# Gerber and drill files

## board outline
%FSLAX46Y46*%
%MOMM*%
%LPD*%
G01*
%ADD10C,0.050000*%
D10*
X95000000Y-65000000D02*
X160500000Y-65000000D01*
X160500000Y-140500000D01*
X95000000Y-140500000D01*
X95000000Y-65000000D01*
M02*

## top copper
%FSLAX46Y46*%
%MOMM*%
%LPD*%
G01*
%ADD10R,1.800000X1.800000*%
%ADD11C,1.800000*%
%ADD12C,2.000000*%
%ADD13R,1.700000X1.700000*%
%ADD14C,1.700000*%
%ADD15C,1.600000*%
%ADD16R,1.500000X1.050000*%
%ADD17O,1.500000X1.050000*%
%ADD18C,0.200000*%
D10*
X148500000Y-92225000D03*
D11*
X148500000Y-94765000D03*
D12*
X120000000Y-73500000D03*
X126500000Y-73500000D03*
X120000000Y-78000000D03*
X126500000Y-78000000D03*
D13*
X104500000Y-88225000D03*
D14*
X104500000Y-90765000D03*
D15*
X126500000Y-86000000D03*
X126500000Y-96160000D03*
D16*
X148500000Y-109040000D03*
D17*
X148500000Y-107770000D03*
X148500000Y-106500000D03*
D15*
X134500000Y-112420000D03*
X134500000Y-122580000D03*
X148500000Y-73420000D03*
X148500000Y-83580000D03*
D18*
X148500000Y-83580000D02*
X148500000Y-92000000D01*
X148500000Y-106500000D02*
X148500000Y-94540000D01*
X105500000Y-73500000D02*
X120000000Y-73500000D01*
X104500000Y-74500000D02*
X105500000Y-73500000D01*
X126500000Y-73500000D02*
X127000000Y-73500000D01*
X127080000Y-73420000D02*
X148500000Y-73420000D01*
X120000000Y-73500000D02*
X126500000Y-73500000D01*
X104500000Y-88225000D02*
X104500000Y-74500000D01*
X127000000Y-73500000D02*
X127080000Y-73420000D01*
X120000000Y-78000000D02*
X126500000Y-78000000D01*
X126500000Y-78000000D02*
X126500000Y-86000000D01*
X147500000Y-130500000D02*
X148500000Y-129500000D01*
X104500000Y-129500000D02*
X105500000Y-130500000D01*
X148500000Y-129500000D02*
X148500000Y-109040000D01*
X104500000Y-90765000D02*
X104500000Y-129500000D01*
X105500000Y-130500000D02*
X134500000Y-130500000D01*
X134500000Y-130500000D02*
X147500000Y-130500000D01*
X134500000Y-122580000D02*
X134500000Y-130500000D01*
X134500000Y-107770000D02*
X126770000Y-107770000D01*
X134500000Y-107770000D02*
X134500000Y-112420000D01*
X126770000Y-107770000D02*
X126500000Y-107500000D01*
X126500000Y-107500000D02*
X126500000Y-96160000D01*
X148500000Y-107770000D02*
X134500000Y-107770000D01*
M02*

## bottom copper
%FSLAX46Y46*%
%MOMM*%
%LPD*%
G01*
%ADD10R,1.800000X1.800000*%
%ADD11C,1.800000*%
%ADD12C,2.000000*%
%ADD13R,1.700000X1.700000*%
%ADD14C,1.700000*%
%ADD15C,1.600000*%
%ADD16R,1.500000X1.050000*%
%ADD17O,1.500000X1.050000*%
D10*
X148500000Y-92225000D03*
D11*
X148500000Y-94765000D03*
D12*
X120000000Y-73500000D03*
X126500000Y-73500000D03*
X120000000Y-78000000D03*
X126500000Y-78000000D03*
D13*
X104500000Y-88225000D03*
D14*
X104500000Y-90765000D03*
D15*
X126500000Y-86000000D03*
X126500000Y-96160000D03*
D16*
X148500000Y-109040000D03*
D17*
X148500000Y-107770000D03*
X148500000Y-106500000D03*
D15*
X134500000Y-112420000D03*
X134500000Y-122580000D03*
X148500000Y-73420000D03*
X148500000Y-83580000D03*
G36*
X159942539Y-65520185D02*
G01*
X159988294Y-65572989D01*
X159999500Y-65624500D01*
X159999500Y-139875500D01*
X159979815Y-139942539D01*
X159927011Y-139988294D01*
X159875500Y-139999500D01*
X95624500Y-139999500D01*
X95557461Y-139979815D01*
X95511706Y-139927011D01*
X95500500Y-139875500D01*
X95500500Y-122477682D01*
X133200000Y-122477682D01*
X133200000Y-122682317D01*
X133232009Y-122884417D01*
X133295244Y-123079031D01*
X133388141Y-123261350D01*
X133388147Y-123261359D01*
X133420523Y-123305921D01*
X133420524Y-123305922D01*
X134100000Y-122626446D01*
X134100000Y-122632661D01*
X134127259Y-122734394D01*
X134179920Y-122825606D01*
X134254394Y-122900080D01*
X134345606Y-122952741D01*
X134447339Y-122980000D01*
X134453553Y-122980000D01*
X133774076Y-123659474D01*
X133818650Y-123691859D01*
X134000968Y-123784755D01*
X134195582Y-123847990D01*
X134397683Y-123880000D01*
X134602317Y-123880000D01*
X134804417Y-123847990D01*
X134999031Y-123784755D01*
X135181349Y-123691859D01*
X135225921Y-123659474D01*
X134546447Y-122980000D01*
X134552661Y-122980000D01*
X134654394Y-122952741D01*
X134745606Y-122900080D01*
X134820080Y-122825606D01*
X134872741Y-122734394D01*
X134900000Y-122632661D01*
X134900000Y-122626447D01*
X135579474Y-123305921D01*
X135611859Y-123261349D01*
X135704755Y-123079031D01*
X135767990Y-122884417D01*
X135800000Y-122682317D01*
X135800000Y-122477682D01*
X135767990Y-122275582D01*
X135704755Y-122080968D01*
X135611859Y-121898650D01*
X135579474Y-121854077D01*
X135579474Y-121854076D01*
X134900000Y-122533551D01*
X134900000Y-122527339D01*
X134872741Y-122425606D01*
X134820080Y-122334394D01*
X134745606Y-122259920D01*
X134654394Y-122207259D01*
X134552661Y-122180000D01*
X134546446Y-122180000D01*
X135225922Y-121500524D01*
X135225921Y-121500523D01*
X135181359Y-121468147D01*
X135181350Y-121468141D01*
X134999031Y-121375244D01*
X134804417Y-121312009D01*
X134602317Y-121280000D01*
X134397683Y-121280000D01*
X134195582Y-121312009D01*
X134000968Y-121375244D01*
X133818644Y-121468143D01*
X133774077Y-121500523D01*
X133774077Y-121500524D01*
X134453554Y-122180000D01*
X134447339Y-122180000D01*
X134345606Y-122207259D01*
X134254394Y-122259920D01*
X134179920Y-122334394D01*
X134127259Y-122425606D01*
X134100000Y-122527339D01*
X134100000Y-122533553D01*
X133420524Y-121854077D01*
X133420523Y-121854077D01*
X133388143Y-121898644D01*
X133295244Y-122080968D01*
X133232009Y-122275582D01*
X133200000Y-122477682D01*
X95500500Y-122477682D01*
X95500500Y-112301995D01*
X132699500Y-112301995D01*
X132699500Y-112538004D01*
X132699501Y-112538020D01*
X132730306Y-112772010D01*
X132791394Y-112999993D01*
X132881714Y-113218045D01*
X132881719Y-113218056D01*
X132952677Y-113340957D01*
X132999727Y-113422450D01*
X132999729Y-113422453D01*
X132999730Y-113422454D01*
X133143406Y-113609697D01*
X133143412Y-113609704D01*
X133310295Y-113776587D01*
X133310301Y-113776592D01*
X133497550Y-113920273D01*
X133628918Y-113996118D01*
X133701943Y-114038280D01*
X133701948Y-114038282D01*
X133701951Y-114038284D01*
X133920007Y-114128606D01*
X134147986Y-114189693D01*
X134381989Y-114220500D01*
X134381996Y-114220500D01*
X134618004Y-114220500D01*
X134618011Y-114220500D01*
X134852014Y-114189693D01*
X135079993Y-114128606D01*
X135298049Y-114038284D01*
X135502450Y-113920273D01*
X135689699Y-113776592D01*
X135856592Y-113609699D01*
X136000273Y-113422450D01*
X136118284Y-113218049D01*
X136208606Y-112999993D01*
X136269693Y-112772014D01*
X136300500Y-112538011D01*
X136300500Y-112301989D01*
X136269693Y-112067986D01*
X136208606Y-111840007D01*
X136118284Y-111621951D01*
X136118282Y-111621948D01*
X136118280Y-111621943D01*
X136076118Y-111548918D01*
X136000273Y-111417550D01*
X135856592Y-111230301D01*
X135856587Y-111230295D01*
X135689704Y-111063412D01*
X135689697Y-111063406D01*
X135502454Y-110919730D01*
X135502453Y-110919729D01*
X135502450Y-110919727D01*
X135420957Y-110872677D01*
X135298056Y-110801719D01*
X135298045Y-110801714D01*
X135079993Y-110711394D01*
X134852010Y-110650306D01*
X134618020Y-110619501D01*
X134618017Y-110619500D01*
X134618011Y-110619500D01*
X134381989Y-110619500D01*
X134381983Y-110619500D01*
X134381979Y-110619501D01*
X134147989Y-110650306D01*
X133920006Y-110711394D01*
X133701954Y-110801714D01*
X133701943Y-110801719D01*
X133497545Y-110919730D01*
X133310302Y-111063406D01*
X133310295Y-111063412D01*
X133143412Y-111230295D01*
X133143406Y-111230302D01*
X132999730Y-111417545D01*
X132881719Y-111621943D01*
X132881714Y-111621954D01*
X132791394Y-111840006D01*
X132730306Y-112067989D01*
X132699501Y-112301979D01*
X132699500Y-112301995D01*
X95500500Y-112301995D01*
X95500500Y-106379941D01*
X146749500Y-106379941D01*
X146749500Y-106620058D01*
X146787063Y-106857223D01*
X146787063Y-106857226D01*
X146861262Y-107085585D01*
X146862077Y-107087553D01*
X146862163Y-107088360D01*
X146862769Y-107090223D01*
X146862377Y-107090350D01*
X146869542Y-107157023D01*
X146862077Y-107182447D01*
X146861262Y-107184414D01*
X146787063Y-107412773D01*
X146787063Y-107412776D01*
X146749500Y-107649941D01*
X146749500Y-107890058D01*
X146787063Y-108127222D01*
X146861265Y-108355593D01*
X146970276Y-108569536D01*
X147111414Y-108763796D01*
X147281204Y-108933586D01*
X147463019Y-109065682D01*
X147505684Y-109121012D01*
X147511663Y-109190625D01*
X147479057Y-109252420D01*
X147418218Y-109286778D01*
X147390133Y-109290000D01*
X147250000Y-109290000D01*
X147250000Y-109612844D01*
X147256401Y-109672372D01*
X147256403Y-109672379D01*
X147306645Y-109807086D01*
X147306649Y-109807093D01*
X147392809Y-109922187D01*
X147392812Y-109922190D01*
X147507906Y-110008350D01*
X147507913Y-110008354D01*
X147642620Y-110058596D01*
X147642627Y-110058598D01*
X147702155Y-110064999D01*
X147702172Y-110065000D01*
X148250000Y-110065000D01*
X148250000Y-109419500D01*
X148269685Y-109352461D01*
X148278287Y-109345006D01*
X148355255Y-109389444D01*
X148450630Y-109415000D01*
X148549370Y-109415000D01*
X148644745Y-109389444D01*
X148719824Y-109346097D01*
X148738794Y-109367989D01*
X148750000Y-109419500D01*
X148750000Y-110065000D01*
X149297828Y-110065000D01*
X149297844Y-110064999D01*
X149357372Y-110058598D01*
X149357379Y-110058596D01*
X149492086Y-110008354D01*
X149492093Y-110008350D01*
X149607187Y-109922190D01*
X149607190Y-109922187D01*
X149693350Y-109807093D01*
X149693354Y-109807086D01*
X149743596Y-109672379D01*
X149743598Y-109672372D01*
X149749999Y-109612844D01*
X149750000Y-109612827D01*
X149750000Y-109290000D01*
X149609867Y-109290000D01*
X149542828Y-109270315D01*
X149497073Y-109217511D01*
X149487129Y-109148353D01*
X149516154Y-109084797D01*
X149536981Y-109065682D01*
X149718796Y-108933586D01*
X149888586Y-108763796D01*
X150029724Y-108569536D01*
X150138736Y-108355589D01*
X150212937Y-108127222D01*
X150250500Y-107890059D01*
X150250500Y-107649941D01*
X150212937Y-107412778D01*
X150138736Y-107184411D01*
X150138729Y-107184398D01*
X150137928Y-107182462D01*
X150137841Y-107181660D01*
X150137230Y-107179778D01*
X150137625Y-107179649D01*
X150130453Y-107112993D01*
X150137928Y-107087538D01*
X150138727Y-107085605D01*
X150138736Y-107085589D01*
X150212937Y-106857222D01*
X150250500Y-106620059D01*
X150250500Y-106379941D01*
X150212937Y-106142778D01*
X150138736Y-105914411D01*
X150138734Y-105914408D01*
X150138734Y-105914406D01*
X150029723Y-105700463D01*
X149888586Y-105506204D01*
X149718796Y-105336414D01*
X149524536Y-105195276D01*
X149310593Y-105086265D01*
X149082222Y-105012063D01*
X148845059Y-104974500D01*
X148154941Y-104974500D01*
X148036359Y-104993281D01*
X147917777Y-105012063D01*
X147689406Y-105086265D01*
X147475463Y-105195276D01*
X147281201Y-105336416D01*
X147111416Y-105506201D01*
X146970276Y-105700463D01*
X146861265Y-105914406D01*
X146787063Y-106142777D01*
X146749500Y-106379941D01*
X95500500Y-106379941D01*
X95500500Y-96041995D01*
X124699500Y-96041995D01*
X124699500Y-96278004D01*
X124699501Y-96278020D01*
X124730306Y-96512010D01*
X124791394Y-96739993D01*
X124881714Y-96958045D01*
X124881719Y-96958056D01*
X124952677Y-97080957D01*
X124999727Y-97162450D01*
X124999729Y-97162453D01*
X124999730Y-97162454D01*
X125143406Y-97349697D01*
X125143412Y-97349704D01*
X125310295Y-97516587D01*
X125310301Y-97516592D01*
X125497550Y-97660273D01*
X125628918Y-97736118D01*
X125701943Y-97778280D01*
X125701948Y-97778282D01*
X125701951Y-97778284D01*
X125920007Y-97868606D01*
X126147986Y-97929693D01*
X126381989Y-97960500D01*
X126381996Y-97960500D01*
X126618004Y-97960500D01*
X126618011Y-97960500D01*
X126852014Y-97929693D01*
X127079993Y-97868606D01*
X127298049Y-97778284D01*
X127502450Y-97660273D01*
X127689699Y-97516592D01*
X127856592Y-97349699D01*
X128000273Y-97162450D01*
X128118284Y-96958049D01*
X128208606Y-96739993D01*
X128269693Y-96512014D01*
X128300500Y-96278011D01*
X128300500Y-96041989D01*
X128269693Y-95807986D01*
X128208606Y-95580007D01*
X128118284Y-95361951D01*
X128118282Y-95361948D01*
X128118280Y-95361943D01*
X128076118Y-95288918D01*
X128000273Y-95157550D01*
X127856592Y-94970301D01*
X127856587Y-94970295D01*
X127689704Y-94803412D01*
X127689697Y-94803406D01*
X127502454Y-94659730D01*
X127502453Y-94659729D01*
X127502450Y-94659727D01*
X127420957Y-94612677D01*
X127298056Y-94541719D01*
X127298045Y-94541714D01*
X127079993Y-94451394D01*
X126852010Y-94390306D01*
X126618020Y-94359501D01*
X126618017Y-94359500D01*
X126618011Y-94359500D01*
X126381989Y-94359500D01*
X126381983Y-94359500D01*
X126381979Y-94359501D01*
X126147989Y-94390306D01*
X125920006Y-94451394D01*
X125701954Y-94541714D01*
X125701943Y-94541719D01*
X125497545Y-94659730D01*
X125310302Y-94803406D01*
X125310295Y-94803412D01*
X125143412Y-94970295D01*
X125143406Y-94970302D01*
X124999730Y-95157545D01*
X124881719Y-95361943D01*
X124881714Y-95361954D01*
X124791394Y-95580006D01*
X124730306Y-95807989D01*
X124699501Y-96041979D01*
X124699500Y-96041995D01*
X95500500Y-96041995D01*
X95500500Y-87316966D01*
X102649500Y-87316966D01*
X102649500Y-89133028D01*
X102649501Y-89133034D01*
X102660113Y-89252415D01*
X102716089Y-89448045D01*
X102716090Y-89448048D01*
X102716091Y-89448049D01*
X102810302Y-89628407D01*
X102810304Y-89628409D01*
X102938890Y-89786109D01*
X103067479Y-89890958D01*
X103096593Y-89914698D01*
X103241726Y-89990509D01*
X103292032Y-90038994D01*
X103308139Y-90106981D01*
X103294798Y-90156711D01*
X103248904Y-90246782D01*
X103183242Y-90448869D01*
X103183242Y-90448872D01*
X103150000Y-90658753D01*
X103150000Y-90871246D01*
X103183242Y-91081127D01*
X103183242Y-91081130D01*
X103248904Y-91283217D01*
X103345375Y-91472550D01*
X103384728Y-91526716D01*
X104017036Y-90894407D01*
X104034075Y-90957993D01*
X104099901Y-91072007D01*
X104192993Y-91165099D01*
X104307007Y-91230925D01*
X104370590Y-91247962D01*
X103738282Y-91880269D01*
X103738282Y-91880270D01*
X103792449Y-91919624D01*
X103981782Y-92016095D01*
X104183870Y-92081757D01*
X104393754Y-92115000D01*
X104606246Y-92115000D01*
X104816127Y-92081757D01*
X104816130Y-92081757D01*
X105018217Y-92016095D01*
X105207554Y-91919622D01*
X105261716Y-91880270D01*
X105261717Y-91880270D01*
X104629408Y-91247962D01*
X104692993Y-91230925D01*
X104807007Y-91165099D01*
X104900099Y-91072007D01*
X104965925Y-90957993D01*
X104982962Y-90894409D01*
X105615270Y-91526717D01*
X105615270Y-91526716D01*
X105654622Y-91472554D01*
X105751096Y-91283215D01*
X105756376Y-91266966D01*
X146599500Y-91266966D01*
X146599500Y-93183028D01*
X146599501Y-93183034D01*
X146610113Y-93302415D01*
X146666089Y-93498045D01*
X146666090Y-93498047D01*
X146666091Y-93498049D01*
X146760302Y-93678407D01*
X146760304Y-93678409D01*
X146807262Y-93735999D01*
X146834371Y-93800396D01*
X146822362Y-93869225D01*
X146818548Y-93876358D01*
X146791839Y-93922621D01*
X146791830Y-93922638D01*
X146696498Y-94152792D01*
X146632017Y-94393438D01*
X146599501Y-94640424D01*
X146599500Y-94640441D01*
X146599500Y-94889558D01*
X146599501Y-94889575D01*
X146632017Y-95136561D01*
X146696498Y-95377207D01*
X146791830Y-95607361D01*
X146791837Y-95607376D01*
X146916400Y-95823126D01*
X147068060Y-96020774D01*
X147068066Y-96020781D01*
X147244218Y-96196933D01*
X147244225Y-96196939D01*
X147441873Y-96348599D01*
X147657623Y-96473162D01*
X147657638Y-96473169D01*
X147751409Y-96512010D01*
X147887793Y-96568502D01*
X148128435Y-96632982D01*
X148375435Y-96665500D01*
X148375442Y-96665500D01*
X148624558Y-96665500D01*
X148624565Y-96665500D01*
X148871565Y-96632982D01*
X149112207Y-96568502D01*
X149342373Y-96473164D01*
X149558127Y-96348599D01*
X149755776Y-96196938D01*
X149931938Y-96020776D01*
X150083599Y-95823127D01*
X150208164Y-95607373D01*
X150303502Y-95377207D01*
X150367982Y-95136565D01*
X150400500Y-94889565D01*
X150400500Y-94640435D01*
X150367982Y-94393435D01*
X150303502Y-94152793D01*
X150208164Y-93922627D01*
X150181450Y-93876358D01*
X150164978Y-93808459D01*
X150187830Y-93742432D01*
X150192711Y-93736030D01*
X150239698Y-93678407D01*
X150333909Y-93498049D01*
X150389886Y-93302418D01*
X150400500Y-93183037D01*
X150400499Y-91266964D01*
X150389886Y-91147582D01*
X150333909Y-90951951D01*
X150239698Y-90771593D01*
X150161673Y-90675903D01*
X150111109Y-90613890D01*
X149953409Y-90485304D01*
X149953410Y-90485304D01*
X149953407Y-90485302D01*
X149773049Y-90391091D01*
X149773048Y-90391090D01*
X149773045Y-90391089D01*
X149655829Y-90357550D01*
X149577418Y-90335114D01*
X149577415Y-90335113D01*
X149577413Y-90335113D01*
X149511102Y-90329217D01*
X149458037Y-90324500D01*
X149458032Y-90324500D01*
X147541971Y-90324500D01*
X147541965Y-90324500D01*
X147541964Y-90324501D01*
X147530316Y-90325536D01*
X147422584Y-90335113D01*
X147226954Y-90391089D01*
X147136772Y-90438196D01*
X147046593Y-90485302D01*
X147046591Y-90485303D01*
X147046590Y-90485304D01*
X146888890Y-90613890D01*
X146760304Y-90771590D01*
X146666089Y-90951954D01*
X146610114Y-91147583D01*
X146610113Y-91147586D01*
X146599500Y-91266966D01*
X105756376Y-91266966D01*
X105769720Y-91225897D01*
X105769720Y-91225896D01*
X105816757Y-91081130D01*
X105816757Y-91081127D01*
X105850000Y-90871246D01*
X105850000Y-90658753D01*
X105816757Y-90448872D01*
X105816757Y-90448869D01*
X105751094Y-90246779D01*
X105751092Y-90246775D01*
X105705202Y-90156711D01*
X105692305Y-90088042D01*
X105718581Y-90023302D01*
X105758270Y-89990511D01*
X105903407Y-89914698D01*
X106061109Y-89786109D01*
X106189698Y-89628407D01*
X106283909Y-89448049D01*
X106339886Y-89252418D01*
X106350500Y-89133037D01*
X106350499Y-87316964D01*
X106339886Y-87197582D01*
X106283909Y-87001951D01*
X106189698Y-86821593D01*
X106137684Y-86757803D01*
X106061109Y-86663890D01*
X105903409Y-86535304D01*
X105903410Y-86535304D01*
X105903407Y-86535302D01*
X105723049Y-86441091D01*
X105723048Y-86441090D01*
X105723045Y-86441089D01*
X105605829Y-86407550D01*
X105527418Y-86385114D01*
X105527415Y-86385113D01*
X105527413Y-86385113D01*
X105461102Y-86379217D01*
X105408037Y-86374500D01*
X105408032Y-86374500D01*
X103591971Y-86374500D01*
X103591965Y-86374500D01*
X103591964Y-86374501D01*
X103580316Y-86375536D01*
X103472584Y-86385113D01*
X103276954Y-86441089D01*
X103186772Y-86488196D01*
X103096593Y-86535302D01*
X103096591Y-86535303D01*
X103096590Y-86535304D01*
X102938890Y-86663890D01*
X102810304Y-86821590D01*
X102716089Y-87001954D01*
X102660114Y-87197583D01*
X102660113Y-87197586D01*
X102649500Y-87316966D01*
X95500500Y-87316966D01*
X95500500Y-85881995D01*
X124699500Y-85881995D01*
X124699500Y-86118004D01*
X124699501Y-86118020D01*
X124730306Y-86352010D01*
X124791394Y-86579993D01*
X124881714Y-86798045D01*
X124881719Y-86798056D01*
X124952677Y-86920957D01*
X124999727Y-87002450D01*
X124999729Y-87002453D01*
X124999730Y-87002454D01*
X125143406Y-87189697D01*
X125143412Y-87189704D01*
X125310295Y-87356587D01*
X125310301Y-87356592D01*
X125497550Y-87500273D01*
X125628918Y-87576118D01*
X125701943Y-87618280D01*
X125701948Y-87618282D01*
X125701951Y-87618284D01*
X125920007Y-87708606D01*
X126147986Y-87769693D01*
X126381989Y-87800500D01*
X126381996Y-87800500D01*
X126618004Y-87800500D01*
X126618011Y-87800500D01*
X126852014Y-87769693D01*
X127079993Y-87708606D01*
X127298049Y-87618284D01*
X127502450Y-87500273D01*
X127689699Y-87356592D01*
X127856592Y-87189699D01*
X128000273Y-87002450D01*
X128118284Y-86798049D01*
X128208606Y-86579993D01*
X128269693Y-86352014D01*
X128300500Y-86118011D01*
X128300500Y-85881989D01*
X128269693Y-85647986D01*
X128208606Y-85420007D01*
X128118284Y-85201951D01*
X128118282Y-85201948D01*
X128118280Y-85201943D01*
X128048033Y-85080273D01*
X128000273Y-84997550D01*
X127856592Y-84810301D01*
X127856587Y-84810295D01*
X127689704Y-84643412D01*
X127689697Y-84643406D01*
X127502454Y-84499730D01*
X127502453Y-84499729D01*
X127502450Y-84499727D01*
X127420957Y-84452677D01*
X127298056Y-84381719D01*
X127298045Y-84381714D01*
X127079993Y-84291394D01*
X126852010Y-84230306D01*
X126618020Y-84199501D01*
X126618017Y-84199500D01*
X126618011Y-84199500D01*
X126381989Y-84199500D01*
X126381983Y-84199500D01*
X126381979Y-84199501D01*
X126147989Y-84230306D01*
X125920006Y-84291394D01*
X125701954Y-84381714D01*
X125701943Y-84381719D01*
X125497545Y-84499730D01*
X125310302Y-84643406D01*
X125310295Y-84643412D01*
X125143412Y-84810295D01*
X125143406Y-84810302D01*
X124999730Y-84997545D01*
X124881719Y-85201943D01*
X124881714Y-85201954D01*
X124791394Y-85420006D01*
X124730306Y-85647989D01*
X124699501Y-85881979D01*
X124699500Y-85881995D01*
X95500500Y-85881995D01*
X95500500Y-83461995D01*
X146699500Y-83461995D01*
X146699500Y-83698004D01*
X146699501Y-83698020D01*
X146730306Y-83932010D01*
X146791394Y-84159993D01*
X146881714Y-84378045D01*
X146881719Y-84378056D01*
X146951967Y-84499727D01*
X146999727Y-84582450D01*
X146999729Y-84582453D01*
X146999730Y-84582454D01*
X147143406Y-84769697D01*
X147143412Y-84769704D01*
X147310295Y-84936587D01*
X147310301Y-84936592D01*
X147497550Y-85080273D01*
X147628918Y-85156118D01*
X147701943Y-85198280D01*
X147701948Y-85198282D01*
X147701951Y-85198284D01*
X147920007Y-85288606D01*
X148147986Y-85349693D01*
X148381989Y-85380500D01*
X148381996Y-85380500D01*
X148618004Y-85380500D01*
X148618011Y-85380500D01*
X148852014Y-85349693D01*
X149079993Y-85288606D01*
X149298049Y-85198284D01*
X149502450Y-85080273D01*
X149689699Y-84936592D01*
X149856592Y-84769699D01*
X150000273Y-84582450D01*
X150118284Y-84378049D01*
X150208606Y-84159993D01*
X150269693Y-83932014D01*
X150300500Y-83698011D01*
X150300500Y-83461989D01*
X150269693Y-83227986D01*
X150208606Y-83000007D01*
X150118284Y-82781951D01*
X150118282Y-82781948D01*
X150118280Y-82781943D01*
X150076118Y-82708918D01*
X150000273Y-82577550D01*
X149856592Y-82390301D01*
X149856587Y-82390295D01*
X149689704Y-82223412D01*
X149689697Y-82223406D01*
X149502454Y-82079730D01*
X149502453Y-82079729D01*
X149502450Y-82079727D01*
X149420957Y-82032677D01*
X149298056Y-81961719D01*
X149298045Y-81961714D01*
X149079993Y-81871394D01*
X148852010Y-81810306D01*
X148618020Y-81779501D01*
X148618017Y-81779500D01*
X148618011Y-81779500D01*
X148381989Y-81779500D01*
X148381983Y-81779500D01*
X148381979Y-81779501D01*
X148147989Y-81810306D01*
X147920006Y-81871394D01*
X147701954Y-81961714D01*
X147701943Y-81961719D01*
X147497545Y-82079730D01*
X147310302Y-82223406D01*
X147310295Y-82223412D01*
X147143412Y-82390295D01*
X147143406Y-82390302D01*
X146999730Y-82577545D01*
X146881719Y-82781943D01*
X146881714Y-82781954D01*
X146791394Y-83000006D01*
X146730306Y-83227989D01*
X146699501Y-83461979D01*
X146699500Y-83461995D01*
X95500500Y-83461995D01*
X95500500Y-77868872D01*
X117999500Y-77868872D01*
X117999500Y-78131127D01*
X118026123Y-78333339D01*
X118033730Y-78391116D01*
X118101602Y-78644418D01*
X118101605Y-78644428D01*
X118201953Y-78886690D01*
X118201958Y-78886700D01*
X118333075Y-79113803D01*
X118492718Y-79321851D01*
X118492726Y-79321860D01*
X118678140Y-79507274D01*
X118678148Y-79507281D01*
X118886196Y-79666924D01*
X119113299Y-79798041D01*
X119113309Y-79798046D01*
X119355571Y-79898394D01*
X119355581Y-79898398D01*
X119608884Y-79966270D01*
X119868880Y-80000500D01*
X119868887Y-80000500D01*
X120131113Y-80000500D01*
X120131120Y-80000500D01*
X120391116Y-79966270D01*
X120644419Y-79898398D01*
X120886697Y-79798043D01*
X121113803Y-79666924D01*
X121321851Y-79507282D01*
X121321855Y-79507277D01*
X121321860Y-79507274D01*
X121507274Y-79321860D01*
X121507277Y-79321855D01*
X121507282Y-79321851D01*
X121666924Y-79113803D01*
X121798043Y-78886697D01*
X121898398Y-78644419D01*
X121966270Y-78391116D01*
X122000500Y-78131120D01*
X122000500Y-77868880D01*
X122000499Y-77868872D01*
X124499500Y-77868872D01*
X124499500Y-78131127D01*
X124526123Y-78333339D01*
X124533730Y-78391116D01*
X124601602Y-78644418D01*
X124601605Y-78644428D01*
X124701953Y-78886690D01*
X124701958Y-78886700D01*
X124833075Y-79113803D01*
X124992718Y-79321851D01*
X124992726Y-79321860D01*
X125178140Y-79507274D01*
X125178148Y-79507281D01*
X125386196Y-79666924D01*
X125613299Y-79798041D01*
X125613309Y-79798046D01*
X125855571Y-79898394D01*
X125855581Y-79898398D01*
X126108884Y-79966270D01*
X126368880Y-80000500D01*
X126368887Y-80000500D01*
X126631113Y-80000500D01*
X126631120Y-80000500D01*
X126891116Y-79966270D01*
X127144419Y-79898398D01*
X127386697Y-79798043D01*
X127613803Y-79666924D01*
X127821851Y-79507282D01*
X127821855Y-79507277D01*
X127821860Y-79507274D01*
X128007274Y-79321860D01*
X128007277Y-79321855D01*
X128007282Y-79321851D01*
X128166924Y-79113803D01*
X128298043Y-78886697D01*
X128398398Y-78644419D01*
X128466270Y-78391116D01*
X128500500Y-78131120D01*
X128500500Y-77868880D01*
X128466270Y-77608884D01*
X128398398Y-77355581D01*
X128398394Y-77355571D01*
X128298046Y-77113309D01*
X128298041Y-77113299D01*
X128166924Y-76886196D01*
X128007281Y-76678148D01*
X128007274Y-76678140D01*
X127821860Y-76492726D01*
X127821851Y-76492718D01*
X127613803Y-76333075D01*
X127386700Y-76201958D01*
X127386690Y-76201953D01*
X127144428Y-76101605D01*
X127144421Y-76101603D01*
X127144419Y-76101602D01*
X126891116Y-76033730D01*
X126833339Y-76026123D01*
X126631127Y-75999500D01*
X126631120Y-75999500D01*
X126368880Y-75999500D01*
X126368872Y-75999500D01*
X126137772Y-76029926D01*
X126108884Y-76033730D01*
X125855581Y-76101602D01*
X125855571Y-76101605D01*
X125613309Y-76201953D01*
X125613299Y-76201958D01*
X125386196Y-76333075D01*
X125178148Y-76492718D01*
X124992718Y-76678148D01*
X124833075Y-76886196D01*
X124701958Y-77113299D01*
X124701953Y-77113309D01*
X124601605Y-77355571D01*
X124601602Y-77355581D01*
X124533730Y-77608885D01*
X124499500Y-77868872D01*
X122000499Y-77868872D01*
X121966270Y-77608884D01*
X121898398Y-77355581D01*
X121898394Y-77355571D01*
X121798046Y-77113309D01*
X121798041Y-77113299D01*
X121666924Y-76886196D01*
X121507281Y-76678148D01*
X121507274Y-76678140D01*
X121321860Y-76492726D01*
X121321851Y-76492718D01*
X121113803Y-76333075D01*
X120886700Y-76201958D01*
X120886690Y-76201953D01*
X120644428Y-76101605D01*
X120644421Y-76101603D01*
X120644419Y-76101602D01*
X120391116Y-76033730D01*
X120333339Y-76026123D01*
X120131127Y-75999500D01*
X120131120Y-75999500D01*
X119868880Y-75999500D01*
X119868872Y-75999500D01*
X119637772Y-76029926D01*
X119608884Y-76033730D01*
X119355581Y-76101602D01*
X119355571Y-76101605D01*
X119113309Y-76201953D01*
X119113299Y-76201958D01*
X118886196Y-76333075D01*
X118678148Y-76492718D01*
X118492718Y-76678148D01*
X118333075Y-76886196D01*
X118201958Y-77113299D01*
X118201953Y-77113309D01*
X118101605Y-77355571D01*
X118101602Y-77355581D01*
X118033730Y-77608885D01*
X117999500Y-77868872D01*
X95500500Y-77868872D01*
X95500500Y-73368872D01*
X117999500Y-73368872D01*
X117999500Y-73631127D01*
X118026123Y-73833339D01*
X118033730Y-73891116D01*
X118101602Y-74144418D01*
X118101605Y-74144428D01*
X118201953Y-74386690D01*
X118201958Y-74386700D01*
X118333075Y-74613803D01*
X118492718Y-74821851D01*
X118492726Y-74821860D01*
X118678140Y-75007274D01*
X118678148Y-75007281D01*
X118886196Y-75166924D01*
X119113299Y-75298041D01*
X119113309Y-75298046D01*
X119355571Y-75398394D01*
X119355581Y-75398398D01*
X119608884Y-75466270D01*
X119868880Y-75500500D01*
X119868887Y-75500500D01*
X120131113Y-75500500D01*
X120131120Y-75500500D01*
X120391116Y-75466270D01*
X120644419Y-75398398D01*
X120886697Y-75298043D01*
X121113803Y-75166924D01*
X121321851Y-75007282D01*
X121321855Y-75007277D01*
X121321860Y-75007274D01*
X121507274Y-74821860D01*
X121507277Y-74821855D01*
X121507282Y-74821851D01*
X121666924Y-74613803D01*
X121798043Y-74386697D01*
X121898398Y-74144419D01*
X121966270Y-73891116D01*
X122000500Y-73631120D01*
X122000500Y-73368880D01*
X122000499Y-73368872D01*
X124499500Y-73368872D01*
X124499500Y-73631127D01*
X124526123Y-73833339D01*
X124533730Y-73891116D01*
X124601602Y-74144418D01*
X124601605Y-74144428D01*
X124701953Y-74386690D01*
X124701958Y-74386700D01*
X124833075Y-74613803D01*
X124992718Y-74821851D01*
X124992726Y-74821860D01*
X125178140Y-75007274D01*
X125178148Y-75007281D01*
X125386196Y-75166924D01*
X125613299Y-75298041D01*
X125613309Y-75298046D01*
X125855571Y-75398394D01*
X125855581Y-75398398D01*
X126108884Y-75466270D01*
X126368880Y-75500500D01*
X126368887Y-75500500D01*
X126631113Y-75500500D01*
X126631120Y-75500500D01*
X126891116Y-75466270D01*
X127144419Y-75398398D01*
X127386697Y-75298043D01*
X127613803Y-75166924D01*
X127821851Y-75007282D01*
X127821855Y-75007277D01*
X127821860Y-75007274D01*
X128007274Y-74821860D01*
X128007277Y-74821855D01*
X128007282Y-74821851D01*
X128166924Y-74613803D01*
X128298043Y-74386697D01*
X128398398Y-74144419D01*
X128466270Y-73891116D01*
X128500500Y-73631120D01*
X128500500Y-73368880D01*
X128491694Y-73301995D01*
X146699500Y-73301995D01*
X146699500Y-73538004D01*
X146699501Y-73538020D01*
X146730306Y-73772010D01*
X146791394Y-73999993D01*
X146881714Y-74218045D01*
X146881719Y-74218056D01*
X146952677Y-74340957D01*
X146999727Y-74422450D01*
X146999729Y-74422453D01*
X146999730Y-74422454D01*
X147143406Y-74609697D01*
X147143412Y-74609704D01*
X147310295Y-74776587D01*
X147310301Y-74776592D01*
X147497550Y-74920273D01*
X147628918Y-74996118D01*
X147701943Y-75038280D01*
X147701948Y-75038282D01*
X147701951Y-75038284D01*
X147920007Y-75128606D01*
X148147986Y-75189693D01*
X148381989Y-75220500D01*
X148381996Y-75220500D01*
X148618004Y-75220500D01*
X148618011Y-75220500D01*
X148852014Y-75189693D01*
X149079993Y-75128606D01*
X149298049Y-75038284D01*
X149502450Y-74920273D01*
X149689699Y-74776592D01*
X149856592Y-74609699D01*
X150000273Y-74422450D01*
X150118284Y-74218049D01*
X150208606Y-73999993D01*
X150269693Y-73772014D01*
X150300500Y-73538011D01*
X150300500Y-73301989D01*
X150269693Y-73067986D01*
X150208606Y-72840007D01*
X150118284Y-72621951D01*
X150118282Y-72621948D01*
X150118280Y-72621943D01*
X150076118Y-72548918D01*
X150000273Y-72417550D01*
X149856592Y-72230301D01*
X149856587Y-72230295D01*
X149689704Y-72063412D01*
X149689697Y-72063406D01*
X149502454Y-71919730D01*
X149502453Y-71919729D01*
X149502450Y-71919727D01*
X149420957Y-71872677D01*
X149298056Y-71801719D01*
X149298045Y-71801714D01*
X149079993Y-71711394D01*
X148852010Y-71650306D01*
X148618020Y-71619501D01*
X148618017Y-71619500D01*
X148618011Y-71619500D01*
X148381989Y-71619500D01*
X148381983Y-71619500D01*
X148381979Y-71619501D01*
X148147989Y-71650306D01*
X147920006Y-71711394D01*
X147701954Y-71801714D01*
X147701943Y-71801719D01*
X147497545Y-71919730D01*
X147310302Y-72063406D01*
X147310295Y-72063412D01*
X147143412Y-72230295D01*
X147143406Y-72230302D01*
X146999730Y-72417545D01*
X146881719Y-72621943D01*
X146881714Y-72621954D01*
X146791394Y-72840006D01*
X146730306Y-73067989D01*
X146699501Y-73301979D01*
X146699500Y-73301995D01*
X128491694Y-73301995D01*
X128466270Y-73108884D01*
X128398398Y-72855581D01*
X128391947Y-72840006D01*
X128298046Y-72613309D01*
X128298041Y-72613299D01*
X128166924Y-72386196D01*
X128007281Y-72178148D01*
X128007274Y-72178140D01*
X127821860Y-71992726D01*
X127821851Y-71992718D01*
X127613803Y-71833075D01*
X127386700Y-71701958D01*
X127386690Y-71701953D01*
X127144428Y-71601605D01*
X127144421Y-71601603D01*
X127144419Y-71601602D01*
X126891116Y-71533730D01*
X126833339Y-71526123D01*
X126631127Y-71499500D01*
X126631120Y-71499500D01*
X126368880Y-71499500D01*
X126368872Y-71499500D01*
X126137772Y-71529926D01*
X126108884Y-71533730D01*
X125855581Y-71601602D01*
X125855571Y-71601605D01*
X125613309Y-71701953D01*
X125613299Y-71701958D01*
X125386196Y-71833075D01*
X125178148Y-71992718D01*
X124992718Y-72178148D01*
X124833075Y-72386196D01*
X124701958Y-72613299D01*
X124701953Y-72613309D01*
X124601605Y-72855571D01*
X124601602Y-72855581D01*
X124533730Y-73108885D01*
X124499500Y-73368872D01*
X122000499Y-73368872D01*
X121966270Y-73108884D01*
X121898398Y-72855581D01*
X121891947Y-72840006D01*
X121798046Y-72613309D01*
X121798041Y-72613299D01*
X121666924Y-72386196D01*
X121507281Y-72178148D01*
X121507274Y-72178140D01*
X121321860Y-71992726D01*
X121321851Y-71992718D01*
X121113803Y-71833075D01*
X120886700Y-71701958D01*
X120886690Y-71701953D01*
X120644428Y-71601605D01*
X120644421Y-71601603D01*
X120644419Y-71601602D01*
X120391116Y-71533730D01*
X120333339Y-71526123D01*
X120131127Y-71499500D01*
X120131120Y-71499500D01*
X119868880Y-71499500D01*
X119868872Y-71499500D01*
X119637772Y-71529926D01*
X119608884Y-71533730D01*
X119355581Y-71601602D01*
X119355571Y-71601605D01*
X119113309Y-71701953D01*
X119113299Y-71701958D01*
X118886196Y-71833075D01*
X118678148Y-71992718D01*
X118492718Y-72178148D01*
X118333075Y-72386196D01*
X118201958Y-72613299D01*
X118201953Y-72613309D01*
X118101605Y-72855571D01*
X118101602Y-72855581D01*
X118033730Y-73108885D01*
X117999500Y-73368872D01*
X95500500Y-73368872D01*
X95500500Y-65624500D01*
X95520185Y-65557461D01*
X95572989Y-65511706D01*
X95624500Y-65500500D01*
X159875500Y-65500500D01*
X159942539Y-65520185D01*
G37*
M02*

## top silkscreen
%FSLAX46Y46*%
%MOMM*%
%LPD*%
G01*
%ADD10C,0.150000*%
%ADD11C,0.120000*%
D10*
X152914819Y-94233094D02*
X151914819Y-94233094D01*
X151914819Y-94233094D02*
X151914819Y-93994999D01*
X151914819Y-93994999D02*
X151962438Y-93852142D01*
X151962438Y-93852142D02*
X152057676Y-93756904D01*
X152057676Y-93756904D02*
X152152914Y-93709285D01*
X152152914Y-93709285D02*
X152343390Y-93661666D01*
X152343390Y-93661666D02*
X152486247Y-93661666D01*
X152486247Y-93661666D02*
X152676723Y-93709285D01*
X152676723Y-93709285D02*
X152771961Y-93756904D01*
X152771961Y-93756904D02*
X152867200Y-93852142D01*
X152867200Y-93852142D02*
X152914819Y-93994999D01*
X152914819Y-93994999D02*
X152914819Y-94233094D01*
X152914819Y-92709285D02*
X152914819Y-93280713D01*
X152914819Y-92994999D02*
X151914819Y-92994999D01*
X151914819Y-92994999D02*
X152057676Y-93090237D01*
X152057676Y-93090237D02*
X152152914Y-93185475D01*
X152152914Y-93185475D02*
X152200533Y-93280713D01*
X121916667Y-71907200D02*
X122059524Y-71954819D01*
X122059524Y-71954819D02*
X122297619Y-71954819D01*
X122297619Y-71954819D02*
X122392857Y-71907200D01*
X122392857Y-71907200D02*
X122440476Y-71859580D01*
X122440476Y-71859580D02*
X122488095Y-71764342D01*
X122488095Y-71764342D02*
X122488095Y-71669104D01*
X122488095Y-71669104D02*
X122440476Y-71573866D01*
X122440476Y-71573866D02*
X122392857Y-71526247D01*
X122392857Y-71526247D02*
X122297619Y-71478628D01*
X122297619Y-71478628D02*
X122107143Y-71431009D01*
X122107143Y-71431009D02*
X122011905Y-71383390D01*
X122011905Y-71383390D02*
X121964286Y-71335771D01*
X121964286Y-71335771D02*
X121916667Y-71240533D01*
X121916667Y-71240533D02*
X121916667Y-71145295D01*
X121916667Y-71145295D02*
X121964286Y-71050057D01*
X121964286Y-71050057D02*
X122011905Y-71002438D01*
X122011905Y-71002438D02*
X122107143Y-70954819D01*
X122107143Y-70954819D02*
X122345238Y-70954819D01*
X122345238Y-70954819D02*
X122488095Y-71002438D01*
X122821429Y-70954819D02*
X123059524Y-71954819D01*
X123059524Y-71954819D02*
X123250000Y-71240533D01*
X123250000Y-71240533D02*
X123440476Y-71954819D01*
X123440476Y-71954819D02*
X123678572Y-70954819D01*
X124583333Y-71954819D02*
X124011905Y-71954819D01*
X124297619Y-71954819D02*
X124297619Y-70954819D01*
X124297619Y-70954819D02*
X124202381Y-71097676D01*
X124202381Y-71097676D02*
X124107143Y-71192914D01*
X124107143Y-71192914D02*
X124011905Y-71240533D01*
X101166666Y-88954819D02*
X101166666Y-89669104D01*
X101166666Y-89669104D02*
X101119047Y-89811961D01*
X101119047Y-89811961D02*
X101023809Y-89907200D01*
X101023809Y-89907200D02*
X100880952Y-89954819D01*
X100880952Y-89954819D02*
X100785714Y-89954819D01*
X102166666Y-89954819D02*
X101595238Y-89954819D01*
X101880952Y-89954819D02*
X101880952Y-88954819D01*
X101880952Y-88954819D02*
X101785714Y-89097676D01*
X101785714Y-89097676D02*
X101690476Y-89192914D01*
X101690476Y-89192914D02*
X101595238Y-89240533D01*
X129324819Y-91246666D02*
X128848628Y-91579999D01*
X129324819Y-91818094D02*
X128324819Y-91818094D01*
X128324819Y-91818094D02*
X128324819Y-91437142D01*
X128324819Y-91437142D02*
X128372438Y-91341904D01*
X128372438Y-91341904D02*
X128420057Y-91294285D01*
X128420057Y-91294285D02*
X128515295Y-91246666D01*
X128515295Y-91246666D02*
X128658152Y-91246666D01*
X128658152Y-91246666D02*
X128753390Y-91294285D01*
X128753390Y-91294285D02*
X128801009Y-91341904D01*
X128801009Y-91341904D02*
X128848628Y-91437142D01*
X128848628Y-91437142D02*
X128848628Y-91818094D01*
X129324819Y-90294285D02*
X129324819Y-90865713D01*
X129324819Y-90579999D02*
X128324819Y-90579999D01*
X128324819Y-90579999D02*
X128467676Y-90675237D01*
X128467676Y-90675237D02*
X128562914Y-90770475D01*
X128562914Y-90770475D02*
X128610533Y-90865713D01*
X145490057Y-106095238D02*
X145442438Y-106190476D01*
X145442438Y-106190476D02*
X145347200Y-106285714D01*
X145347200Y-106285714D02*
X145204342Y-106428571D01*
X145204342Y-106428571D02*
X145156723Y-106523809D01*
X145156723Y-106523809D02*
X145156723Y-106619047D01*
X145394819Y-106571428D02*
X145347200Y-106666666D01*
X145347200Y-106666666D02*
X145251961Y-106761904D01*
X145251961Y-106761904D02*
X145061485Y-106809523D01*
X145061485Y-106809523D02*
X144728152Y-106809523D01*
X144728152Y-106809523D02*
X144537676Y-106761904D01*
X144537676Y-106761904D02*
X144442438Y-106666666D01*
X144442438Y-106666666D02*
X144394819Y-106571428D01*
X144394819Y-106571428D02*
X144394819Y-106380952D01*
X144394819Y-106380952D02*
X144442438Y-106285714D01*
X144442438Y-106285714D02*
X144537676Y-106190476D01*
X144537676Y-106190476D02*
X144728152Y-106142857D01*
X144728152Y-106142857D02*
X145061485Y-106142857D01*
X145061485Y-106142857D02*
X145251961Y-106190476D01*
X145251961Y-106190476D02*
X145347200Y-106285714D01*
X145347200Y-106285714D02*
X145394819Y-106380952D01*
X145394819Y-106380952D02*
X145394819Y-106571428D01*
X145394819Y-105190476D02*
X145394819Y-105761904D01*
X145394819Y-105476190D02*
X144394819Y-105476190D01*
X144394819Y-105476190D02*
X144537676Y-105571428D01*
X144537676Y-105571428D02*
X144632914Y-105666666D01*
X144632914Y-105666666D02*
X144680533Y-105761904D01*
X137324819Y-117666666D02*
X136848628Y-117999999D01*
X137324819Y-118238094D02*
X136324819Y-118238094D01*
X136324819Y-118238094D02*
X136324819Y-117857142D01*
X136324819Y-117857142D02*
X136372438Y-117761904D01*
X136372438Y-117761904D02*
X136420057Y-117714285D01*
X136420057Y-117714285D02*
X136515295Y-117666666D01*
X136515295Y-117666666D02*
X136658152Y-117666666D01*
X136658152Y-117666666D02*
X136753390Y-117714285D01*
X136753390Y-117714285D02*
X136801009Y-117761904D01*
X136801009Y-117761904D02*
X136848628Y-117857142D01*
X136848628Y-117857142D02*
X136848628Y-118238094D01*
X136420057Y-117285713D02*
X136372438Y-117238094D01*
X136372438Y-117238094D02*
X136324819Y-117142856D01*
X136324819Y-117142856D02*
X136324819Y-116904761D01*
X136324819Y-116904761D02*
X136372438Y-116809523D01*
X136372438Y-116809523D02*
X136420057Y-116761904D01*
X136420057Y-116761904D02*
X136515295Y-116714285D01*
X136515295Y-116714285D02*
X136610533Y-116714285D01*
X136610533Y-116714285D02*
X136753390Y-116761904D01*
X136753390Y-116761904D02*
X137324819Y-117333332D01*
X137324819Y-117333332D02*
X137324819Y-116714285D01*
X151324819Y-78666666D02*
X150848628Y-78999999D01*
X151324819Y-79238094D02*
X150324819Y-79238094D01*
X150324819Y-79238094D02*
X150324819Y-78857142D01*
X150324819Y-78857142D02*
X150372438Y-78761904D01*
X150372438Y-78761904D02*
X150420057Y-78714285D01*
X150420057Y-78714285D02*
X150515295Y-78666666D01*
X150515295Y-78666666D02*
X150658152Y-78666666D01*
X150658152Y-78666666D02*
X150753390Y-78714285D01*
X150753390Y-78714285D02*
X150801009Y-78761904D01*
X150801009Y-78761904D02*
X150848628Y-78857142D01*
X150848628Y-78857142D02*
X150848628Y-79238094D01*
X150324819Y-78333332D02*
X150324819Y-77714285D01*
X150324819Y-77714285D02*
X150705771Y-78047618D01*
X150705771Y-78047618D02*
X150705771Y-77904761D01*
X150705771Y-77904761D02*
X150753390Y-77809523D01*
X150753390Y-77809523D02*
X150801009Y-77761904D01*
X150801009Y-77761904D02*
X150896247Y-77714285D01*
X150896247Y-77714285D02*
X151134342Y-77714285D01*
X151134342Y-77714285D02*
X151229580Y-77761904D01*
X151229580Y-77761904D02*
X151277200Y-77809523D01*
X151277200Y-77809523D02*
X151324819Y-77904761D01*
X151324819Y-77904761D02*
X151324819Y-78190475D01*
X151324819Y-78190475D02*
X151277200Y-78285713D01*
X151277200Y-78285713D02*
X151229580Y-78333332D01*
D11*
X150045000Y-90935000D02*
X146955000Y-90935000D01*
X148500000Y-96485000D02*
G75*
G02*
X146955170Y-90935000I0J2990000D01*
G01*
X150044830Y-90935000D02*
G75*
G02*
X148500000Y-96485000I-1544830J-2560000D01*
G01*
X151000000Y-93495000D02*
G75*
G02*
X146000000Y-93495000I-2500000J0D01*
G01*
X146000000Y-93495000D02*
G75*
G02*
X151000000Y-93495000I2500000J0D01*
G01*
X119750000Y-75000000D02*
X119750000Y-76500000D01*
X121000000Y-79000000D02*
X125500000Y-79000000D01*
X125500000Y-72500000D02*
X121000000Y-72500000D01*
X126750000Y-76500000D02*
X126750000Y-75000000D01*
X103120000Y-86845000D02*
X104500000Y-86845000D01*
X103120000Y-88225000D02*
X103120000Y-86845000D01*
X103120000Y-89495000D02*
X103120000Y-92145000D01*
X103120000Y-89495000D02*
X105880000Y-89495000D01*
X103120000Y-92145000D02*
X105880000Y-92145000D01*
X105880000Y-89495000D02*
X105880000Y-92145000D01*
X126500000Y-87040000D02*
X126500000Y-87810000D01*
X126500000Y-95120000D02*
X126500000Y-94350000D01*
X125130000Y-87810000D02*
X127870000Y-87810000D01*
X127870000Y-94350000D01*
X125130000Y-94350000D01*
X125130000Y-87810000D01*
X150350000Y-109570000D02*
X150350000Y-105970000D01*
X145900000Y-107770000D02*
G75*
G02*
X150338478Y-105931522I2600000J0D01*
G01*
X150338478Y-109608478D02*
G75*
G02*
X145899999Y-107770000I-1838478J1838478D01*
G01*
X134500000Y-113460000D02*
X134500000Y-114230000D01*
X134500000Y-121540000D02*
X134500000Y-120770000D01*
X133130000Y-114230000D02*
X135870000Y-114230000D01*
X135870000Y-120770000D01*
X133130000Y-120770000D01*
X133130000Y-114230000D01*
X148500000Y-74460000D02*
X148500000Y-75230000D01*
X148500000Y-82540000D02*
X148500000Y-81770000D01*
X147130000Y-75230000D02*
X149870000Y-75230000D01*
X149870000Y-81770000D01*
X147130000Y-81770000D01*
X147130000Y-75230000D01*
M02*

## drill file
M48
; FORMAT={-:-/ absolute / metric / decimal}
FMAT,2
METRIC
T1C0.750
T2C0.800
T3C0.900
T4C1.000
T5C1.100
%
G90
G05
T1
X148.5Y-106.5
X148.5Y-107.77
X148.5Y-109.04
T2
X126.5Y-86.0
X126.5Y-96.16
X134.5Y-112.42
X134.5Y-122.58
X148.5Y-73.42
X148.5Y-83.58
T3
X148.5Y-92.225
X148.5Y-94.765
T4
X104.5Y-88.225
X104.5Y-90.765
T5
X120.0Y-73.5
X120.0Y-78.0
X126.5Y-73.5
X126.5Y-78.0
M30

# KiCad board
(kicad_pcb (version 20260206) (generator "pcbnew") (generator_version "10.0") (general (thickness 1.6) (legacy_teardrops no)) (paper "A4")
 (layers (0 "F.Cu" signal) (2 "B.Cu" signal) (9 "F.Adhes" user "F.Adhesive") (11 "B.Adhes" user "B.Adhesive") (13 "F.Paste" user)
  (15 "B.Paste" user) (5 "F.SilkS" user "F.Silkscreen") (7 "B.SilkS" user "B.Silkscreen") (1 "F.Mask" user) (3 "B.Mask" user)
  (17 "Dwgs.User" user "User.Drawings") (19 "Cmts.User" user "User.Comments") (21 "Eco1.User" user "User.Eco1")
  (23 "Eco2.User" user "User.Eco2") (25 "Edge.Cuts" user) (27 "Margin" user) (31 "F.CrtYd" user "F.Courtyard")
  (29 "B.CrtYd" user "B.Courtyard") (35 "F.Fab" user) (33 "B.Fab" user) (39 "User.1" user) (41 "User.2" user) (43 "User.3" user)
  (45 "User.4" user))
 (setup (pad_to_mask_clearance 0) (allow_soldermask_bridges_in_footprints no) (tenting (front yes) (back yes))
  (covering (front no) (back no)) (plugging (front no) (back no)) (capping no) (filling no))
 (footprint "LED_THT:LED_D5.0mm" (layer "F.Cu") (at 148.5 92.225 -90)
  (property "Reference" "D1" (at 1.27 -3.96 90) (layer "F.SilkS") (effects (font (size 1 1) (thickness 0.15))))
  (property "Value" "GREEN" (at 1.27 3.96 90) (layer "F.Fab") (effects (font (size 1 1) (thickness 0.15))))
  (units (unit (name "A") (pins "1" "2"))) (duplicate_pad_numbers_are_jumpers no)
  (fp_line (start -1.29 -1.545) (end -1.29 1.545) (stroke (width 0.12) (type solid)) (layer "F.SilkS"))
  (fp_arc (start 4.26 0) (mid 2.071779 2.880495) (end -1.29 1.54483) (stroke (width 0.12) (type solid)) (layer "F.SilkS"))
  (fp_arc (start -1.29 -1.54483) (mid 2.071779 -2.880495) (end 4.26 0) (stroke (width 0.12) (type solid)) (layer "F.SilkS"))
  (fp_circle (center 1.27 0) (end 3.77 0) (stroke (width 0.12) (type solid)) (fill no) (layer "F.SilkS"))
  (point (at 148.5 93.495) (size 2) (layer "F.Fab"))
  (pad "1" thru_hole rect (at 0 0 270) (size 1.8 1.8) (drill 0.9) (layers "*.Cu" "*.Mask") (remove_unused_layers no) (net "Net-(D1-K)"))
  (pad "2" thru_hole circle (at 2.54 0 270) (size 1.8 1.8) (drill 0.9) (layers "*.Cu" "*.Mask") (remove_unused_layers no) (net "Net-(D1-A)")))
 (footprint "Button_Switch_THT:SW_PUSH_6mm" (layer "F.Cu") (at 120 73.5)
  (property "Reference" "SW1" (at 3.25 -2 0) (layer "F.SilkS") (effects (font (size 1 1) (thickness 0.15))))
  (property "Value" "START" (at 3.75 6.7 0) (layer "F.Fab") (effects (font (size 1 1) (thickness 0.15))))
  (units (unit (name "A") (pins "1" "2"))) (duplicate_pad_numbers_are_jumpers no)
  (fp_line (start -0.25 1.5) (end -0.25 3) (stroke (width 0.12) (type solid)) (layer "F.SilkS"))
  (fp_line (start 1 5.5) (end 5.5 5.5) (stroke (width 0.12) (type solid)) (layer "F.SilkS"))
  (fp_line (start 5.5 -1) (end 1 -1) (stroke (width 0.12) (type solid)) (layer "F.SilkS"))
  (fp_line (start 6.75 3) (end 6.75 1.5) (stroke (width 0.12) (type solid)) (layer "F.SilkS"))
  (pad "1" thru_hole circle (at 0 0 90) (size 2 2) (drill 1.1) (layers "*.Cu" "*.Mask") (remove_unused_layers no) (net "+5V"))
  (pad "1" thru_hole circle (at 6.5 0 90) (size 2 2) (drill 1.1) (layers "*.Cu" "*.Mask") (remove_unused_layers no) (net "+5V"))
  (pad "2" thru_hole circle (at 0 4.5 90) (size 2 2) (drill 1.1) (layers "*.Cu" "*.Mask") (remove_unused_layers no) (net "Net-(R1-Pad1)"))
  (pad "2" thru_hole circle (at 6.5 4.5 90) (size 2 2) (drill 1.1) (layers "*.Cu" "*.Mask") (remove_unused_layers no) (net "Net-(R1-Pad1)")))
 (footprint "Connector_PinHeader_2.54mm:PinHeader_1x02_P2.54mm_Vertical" (layer "F.Cu") (at 104.5 88.225)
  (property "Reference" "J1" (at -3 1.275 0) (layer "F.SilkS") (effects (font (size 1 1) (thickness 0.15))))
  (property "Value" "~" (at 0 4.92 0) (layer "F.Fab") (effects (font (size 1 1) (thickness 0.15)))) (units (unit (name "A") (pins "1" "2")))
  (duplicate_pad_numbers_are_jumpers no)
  (fp_line (start -1.38 -1.38) (end 0 -1.38) (stroke (width 0.12) (type solid)) (layer "F.SilkS"))
  (fp_line (start -1.38 0) (end -1.38 -1.38) (stroke (width 0.12) (type solid)) (layer "F.SilkS"))
  (fp_line (start -1.38 1.27) (end -1.38 3.92) (stroke (width 0.12) (type solid)) (layer "F.SilkS"))
  (fp_line (start -1.38 1.27) (end 1.38 1.27) (stroke (width 0.12) (type solid)) (layer "F.SilkS"))
  (fp_line (start -1.38 3.92) (end 1.38 3.92) (stroke (width 0.12) (type solid)) (layer "F.SilkS"))
  (fp_line (start 1.38 1.27) (end 1.38 3.92) (stroke (width 0.12) (type solid)) (layer "F.SilkS"))
  (pad "1" thru_hole rect (at 0 0) (size 1.7 1.7) (drill 1) (layers "*.Cu" "*.Mask") (remove_unused_layers no) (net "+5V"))
  (pad "2" thru_hole circle (at 0 2.54) (size 1.7 1.7) (drill 1) (layers "*.Cu" "*.Mask") (remove_unused_layers no) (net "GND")))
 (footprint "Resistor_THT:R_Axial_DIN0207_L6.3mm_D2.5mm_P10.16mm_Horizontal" (layer "F.Cu") (at 126.5 86 -90)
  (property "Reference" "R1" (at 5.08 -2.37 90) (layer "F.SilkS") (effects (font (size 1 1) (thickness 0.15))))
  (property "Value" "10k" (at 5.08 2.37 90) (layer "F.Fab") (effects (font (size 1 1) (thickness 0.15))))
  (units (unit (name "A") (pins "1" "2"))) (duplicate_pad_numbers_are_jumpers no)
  (fp_line (start 1.04 0) (end 1.81 0) (stroke (width 0.12) (type solid)) (layer "F.SilkS"))
  (fp_line (start 9.12 0) (end 8.35 0) (stroke (width 0.12) (type solid)) (layer "F.SilkS"))
  (fp_rect (start 1.81 -1.37) (end 8.35 1.37) (stroke (width 0.12) (type solid)) (fill no) (layer "F.SilkS"))
  (pad "1" thru_hole circle (at 0 0 270) (size 1.6 1.6) (drill 0.8) (layers "*.Cu" "*.Mask") (remove_unused_layers no) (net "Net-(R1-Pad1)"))
  (pad "2" thru_hole circle (at 10.16 0 270) (size 1.6 1.6) (drill 0.8) (layers "*.Cu" "*.Mask") (remove_unused_layers no) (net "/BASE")))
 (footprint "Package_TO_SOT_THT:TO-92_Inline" (layer "F.Cu") (at 148.5 109.04 90)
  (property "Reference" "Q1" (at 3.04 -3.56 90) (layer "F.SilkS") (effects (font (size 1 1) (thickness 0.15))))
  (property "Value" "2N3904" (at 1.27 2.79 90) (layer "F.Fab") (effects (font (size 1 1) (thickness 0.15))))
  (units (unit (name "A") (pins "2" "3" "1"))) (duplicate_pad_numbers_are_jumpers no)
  (fp_line (start -0.53 1.85) (end 3.07 1.85) (stroke (width 0.12) (type solid)) (layer "F.SilkS"))
  (fp_arc (start 1.27 -2.6) (mid 3.672087 -0.994977) (end 3.108478 1.838478) (stroke (width 0.12) (type solid)) (layer "F.SilkS"))
  (fp_arc (start -0.568478 1.838478) (mid -1.132087 -0.994977) (end 1.27 -2.6) (stroke (width 0.12) (type solid)) (layer "F.SilkS"))
  (pad "1" thru_hole rect (at 0 0 90) (size 1.05 1.5) (drill 0.75) (layers "*.Cu" "*.Mask") (remove_unused_layers no) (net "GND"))
  (pad "2" thru_hole oval (at 1.27 0 90) (size 1.05 1.5) (drill 0.75) (layers "*.Cu" "*.Mask") (remove_unused_layers no) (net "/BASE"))
  (pad "3" thru_hole oval (at 2.54 0 90) (size 1.05 1.5) (drill 0.75) (layers "*.Cu" "*.Mask") (remove_unused_layers no) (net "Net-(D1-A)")))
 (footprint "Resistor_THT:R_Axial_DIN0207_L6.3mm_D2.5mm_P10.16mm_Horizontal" (layer "F.Cu") (at 134.5 112.42 -90)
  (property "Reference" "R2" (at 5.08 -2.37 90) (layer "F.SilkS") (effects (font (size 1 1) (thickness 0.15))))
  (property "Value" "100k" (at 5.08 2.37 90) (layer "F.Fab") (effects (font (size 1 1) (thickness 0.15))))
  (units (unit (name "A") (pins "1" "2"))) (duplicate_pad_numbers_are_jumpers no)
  (fp_line (start 1.04 0) (end 1.81 0) (stroke (width 0.12) (type solid)) (layer "F.SilkS"))
  (fp_line (start 9.12 0) (end 8.35 0) (stroke (width 0.12) (type solid)) (layer "F.SilkS"))
  (fp_rect (start 1.81 -1.37) (end 8.35 1.37) (stroke (width 0.12) (type solid)) (fill no) (layer "F.SilkS"))
  (pad "1" thru_hole circle (at 0 0 270) (size 1.6 1.6) (drill 0.8) (layers "*.Cu" "*.Mask") (remove_unused_layers no) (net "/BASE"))
  (pad "2" thru_hole circle (at 10.16 0 270) (size 1.6 1.6) (drill 0.8) (layers "*.Cu" "*.Mask") (remove_unused_layers no) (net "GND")))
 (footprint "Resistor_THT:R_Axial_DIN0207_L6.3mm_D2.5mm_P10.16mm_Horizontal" (layer "F.Cu") (at 148.5 73.42 -90)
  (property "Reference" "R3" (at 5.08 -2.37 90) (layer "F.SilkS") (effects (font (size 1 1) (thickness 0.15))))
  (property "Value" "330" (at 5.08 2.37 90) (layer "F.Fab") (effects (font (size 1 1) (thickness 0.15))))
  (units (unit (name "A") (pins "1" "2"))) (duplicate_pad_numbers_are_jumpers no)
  (fp_line (start 1.04 0) (end 1.81 0) (stroke (width 0.12) (type solid)) (layer "F.SilkS"))
  (fp_line (start 9.12 0) (end 8.35 0) (stroke (width 0.12) (type solid)) (layer "F.SilkS"))
  (fp_rect (start 1.81 -1.37) (end 8.35 1.37) (stroke (width 0.12) (type solid)) (fill no) (layer "F.SilkS"))
  (pad "1" thru_hole circle (at 0 0 270) (size 1.6 1.6) (drill 0.8) (layers "*.Cu" "*.Mask") (remove_unused_layers no) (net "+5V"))
  (pad "2" thru_hole circle (at 10.16 0 270) (size 1.6 1.6) (drill 0.8) (layers "*.Cu" "*.Mask") (remove_unused_layers no)
   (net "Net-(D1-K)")))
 (gr_rect (start 95 65) (end 160.5 140.5) (stroke (width 0.05) (type default)) (fill no) (layer "Edge.Cuts"))
 (segment (start 148.5 83.58) (end 148.5 92) (width 0.2) (layers "F.Cu" "F.Mask") (solder_mask_margin 0.2) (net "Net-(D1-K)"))
 (segment (start 148.5 106.5) (end 148.5 94.54) (width 0.2) (layers "F.Cu" "F.Mask") (solder_mask_margin 0.2) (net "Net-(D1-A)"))
 (segment (start 105.5 73.5) (end 120 73.5) (width 0.2) (layers "F.Cu" "F.Mask") (solder_mask_margin 0.2) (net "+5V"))
 (segment (start 104.5 74.5) (end 105.5 73.5) (width 0.2) (layers "F.Cu" "F.Mask") (solder_mask_margin 0.2) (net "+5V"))
 (segment (start 126.5 73.5) (end 127 73.5) (width 0.2) (layers "F.Cu" "F.Mask") (solder_mask_margin 0.2) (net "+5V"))
 (segment (start 127.08 73.42) (end 148.5 73.42) (width 0.2) (layers "F.Cu" "F.Mask") (solder_mask_margin 0.2) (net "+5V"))
 (segment (start 120 73.5) (end 126.5 73.5) (width 0.2) (layers "F.Cu" "F.Mask") (solder_mask_margin 0.2) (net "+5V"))
 (segment (start 104.5 88.225) (end 104.5 74.5) (width 0.2) (layers "F.Cu" "F.Mask") (solder_mask_margin 0.2) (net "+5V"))
 (segment (start 127 73.5) (end 127.08 73.42) (width 0.2) (layers "F.Cu" "F.Mask") (solder_mask_margin 0.2) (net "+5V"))
 (segment (start 120 78) (end 126.5 78) (width 0.2) (layers "F.Cu" "F.Mask") (solder_mask_margin 0.2) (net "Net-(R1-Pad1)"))
 (segment (start 126.5 78) (end 126.5 86) (width 0.2) (layers "F.Cu" "F.Mask") (solder_mask_margin 0.2) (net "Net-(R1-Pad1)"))
 (segment (start 147.5 130.5) (end 148.5 129.5) (width 0.2) (layers "F.Cu" "F.Mask") (solder_mask_margin 0.2) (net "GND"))
 (segment (start 104.5 129.5) (end 105.5 130.5) (width 0.2) (layers "F.Cu" "F.Mask") (solder_mask_margin 0.2) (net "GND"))
 (segment (start 148.5 129.5) (end 148.5 109.04) (width 0.2) (layers "F.Cu" "F.Mask") (solder_mask_margin 0.2) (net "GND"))
 (segment (start 104.5 90.765) (end 104.5 129.5) (width 0.2) (layers "F.Cu" "F.Mask") (solder_mask_margin 0.2) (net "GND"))
 (segment (start 105.5 130.5) (end 134.5 130.5) (width 0.2) (layers "F.Cu" "F.Mask") (solder_mask_margin 0.2) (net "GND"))
 (segment (start 134.5 130.5) (end 147.5 130.5) (width 0.2) (layers "F.Cu" "F.Mask") (solder_mask_margin 0.2) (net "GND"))
 (segment (start 134.5 122.58) (end 134.5 130.5) (width 0.2) (layers "F.Cu" "F.Mask") (solder_mask_margin 0.2) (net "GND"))
 (segment (start 134.5 107.77) (end 126.77 107.77) (width 0.2) (layers "F.Cu" "F.Mask") (solder_mask_margin 0.2) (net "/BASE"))
 (segment (start 134.5 107.77) (end 134.5 112.42) (width 0.2) (layers "F.Cu" "F.Mask") (solder_mask_margin 0.2) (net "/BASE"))
 (segment (start 126.77 107.77) (end 126.5 107.5) (width 0.2) (layers "F.Cu" "F.Mask") (solder_mask_margin 0.2) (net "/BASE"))
 (segment (start 126.5 107.5) (end 126.5 96.16) (width 0.2) (layers "F.Cu" "F.Mask") (solder_mask_margin 0.2) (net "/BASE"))
 (segment (start 148.5 107.77) (end 134.5 107.77) (width 0.2) (layers "F.Cu" "F.Mask") (solder_mask_margin 0.2) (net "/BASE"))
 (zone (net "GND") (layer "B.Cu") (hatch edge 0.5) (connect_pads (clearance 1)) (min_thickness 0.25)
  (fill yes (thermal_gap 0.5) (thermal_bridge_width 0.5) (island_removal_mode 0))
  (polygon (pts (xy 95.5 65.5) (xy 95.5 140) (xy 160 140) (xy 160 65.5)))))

